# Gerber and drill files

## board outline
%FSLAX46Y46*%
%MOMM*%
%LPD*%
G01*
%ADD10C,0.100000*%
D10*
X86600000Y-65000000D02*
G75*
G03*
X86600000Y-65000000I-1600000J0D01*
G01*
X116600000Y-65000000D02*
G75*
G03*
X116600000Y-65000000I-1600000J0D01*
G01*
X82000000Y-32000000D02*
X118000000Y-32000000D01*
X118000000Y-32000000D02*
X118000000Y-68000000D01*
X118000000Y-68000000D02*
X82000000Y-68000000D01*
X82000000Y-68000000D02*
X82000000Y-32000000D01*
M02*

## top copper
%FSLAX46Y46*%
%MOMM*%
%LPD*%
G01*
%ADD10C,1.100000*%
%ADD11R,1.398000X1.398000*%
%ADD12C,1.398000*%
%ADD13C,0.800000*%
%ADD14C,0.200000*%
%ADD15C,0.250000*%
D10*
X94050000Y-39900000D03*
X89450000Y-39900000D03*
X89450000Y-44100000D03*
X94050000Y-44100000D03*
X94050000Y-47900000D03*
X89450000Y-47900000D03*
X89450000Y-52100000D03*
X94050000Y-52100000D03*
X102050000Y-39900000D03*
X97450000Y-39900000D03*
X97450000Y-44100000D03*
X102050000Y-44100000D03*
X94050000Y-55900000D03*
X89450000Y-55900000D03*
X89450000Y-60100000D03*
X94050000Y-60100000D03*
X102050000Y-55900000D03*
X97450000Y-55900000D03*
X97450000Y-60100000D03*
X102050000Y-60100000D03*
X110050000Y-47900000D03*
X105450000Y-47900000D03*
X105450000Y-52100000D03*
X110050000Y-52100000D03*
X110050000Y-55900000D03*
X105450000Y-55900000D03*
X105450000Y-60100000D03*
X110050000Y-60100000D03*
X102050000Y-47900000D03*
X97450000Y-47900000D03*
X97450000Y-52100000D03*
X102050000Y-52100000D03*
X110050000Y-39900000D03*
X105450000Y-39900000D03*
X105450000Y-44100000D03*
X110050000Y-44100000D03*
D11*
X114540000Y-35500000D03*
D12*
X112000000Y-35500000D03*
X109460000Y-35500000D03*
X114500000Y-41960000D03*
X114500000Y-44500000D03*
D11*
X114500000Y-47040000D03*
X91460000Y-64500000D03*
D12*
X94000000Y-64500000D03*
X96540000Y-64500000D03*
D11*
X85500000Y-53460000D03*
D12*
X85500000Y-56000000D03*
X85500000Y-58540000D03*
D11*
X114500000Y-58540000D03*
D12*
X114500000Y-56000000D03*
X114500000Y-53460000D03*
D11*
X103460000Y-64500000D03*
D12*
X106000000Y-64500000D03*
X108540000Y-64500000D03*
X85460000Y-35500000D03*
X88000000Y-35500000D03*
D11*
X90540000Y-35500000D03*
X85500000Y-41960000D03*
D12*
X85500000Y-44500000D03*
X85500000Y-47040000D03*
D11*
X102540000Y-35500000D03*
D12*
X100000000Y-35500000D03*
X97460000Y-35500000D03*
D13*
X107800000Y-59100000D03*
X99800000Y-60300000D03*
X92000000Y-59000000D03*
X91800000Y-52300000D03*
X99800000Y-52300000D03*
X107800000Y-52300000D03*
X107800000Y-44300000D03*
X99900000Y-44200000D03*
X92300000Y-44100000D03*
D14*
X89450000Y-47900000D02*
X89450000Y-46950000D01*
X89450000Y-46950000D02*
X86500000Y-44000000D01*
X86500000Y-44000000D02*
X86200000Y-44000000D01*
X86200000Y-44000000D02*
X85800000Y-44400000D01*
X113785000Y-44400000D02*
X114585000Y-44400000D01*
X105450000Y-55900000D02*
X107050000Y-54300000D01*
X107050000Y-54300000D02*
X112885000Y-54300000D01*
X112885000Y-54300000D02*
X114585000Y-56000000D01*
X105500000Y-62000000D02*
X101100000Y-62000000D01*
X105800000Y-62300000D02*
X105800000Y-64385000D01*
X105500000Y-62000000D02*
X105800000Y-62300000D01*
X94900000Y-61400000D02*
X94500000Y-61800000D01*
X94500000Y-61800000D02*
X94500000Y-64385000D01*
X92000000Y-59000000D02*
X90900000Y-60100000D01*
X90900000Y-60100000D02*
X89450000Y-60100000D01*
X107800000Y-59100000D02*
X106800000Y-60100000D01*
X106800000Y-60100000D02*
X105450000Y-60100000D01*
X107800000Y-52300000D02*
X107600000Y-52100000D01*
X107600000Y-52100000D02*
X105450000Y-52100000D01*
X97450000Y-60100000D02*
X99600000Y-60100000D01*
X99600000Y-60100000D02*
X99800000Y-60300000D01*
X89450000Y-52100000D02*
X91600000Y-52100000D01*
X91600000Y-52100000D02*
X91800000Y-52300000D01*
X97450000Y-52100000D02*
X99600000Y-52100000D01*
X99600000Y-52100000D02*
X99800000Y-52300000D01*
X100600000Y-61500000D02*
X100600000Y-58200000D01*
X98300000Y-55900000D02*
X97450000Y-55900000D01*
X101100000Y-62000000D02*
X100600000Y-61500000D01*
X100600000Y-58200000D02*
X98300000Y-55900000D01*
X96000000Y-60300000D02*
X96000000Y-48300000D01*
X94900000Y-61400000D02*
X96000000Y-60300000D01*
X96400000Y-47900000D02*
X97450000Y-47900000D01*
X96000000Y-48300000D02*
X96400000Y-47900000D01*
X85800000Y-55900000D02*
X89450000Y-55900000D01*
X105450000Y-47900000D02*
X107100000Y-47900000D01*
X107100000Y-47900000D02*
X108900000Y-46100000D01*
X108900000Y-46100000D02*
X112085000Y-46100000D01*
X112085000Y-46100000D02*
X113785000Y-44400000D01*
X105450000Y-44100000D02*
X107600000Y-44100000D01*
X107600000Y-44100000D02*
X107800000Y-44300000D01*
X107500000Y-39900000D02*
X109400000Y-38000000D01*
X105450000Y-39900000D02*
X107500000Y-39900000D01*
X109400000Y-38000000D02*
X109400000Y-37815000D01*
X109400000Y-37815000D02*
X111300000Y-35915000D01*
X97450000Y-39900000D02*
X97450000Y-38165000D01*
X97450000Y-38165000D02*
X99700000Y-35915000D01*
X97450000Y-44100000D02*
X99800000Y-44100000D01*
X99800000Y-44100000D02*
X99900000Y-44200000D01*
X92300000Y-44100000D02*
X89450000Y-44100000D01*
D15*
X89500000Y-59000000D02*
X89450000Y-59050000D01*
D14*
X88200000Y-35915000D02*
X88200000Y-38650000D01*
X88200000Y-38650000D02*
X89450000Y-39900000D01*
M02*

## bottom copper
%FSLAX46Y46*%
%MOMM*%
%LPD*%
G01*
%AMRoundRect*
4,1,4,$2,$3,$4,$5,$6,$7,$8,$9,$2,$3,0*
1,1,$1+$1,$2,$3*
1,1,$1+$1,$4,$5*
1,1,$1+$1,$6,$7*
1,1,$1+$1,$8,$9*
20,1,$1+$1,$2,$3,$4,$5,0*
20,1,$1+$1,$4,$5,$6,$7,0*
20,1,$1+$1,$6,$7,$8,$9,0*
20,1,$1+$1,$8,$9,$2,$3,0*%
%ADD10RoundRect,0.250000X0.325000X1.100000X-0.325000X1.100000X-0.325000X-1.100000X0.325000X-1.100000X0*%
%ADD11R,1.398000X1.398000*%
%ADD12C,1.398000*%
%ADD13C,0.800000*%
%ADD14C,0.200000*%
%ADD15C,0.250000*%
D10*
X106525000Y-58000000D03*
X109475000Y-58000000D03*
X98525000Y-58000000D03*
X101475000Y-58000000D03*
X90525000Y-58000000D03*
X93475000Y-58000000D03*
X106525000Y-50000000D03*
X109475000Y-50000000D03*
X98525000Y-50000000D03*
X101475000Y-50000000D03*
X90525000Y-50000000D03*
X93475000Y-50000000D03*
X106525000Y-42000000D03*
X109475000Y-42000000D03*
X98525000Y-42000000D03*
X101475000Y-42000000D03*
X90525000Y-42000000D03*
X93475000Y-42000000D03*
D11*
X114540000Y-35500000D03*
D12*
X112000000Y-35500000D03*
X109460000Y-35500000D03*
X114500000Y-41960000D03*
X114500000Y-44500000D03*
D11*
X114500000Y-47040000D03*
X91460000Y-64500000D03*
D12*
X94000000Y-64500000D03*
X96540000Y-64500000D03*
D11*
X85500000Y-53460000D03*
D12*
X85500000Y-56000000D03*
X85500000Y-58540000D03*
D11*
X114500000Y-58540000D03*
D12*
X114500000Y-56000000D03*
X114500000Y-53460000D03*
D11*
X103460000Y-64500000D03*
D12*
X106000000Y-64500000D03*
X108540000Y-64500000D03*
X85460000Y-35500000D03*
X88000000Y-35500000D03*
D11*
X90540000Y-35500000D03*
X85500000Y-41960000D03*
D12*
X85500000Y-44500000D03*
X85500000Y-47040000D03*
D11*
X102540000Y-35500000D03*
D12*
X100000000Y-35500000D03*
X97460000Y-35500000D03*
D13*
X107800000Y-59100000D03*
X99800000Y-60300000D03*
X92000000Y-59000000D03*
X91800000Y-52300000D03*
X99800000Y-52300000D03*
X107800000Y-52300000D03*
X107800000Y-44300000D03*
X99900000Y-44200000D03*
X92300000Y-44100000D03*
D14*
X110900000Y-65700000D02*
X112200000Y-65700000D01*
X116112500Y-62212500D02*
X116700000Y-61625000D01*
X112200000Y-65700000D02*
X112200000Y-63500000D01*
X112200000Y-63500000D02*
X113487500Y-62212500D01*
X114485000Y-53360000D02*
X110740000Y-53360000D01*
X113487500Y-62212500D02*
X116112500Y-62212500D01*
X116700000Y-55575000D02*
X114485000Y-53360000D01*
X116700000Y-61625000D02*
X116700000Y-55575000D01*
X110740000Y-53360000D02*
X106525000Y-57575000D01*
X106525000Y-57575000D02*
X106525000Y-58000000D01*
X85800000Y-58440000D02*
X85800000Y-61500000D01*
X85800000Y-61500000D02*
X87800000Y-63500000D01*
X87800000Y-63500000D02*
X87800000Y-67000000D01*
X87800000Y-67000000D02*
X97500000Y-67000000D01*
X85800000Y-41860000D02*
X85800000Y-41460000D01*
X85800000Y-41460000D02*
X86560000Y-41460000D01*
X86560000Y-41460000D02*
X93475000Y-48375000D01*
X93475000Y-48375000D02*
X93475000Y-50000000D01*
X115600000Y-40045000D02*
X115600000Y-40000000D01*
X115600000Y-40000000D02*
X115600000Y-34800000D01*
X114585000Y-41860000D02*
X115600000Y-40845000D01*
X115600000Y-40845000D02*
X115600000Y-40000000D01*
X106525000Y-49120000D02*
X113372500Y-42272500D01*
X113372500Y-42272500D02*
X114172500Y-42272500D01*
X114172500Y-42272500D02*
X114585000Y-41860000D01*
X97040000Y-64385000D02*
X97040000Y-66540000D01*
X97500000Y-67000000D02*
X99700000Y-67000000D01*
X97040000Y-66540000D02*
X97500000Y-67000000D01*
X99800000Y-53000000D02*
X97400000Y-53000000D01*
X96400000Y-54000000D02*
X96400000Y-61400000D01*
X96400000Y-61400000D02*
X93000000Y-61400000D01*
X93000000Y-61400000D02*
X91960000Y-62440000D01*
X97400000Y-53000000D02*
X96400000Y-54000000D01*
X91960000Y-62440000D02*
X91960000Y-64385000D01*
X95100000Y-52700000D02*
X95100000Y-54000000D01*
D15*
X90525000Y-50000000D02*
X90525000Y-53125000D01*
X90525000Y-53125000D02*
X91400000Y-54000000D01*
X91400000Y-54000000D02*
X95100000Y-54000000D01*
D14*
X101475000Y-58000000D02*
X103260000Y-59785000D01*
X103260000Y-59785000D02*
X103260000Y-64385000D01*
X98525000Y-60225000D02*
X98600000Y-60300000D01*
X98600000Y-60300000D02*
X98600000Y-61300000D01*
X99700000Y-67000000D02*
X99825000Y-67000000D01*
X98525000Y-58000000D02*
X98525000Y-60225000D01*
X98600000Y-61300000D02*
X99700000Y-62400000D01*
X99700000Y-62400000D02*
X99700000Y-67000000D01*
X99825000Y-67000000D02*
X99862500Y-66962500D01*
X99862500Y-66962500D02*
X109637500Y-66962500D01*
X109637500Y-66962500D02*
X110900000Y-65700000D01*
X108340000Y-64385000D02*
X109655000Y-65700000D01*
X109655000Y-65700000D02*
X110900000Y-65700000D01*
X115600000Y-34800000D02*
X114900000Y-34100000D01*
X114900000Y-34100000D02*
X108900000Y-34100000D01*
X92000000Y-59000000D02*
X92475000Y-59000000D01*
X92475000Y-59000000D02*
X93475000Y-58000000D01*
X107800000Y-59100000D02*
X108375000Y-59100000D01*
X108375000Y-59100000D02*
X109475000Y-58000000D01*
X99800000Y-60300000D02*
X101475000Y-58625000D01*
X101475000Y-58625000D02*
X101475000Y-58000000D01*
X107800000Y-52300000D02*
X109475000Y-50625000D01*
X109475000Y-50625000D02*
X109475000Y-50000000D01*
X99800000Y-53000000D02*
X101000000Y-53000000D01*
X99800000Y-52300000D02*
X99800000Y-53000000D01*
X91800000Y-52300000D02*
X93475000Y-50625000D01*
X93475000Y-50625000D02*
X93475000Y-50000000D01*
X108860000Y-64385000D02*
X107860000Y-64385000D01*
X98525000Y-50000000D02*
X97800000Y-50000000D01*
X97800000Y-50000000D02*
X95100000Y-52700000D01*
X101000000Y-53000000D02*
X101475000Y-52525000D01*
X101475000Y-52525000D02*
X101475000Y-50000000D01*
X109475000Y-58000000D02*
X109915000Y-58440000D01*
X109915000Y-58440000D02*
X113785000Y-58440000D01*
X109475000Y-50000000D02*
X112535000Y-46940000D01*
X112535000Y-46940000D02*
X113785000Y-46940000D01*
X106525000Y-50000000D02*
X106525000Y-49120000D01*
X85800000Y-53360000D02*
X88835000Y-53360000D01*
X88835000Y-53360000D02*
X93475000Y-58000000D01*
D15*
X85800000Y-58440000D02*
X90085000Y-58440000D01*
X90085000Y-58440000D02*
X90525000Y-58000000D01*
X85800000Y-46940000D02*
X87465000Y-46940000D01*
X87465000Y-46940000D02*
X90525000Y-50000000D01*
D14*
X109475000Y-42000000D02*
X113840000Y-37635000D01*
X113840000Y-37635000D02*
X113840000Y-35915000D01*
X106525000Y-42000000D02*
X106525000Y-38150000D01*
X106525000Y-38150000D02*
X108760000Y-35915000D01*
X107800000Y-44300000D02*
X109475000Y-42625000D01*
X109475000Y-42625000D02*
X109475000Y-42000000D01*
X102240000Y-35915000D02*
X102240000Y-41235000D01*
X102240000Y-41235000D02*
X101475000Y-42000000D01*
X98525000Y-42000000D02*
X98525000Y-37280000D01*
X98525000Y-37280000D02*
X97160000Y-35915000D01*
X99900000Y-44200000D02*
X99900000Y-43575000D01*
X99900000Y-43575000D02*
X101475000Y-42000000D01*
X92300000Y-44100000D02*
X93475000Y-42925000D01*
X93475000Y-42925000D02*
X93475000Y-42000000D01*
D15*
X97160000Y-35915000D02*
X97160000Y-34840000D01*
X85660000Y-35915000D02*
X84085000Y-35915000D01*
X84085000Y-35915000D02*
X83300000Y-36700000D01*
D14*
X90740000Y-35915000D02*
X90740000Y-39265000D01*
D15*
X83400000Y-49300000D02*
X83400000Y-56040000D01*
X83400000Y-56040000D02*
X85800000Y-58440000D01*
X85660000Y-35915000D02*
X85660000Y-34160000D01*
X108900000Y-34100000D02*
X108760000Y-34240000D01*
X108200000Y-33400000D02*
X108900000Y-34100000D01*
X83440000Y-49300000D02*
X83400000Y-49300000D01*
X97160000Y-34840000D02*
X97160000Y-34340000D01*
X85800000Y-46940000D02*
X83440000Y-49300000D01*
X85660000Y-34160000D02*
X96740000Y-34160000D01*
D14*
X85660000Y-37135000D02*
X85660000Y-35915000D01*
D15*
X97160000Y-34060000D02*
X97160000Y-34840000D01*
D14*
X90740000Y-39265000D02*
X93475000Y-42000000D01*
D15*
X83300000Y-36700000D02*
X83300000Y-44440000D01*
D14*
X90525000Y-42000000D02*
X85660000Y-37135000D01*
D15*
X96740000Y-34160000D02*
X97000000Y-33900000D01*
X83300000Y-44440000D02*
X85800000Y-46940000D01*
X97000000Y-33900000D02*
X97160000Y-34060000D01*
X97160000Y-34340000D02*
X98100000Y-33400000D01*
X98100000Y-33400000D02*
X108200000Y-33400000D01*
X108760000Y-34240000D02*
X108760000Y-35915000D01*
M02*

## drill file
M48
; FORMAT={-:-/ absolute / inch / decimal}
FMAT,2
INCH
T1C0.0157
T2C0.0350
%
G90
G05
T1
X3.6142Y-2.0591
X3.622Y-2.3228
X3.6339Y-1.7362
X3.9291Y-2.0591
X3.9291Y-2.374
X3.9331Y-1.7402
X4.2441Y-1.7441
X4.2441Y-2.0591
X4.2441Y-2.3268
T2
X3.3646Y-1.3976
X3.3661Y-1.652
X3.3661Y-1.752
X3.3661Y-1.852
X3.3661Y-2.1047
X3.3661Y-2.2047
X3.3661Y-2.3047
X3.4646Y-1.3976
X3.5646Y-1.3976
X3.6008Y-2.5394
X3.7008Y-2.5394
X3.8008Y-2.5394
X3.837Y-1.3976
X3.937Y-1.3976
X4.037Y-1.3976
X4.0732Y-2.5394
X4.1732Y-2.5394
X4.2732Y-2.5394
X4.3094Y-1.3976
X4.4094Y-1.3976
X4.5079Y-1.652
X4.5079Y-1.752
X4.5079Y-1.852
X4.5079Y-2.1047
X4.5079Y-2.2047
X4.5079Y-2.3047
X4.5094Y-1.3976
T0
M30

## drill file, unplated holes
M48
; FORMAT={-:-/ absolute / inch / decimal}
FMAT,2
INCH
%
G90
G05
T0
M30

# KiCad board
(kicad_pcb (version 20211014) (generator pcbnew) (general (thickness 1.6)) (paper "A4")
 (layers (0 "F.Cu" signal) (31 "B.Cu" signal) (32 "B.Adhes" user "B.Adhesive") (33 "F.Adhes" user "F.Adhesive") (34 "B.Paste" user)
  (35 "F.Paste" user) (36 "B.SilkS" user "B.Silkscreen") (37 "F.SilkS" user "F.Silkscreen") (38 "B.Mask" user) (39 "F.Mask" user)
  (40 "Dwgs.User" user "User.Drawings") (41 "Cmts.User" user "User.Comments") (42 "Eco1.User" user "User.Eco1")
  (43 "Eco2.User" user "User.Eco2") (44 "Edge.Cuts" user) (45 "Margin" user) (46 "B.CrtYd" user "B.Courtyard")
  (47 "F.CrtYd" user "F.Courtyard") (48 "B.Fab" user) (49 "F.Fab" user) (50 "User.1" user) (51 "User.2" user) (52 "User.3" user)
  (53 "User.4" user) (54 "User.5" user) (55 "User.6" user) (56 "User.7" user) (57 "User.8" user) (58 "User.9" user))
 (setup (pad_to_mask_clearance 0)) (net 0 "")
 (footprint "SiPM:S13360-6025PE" (layer "F.Cu") (at 92 42)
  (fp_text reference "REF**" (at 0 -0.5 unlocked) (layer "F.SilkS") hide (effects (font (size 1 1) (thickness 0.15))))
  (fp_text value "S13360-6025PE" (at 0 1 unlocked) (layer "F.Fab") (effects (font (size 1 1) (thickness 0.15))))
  (pad "1" smd circle (at 2.05 -2.1) (size 1.1 1.1) (layers "F.Cu" "F.Paste" "F.Mask"))
  (pad "2" smd circle (at -2.55 -2.1) (size 1.1 1.1) (layers "F.Cu" "F.Paste" "F.Mask"))
  (pad "3" smd circle (at -2.55 2.1) (size 1.1 1.1) (layers "F.Cu" "F.Paste" "F.Mask"))
  (pad "4" smd circle (at 2.05 2.1) (size 1.1 1.1) (layers "F.Cu" "F.Paste" "F.Mask")))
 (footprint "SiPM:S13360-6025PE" (layer "F.Cu") (at 92 50)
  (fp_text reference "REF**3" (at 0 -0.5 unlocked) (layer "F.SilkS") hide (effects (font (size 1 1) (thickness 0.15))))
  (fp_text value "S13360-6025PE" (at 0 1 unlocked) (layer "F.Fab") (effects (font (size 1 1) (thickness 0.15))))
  (pad "1" smd circle (at 2.05 -2.1) (size 1.1 1.1) (layers "F.Cu" "F.Paste" "F.Mask"))
  (pad "2" smd circle (at -2.55 -2.1) (size 1.1 1.1) (layers "F.Cu" "F.Paste" "F.Mask"))
  (pad "3" smd circle (at -2.55 2.1) (size 1.1 1.1) (layers "F.Cu" "F.Paste" "F.Mask"))
  (pad "4" smd circle (at 2.05 2.1) (size 1.1 1.1) (layers "F.Cu" "F.Paste" "F.Mask")))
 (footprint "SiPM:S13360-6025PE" (layer "F.Cu") (at 100 42)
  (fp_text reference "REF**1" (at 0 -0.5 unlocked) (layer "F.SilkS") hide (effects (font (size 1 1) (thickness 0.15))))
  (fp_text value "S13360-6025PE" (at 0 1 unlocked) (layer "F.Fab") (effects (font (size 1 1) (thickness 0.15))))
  (pad "1" smd circle (at 2.05 -2.1) (size 1.1 1.1) (layers "F.Cu" "F.Paste" "F.Mask"))
  (pad "2" smd circle (at -2.55 -2.1) (size 1.1 1.1) (layers "F.Cu" "F.Paste" "F.Mask"))
  (pad "3" smd circle (at -2.55 2.1) (size 1.1 1.1) (layers "F.Cu" "F.Paste" "F.Mask"))
  (pad "4" smd circle (at 2.05 2.1) (size 1.1 1.1) (layers "F.Cu" "F.Paste" "F.Mask")))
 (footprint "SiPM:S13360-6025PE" (layer "F.Cu") (at 92 58)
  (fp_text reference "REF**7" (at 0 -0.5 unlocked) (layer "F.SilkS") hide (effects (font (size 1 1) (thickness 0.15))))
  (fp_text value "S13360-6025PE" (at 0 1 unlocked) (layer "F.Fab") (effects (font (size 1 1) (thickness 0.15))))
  (pad "1" smd circle (at 2.05 -2.1) (size 1.1 1.1) (layers "F.Cu" "F.Paste" "F.Mask"))
  (pad "2" smd circle (at -2.55 -2.1) (size 1.1 1.1) (layers "F.Cu" "F.Paste" "F.Mask"))
  (pad "3" smd circle (at -2.55 2.1) (size 1.1 1.1) (layers "F.Cu" "F.Paste" "F.Mask"))
  (pad "4" smd circle (at 2.05 2.1) (size 1.1 1.1) (layers "F.Cu" "F.Paste" "F.Mask")))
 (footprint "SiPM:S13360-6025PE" (layer "F.Cu") (at 100 58)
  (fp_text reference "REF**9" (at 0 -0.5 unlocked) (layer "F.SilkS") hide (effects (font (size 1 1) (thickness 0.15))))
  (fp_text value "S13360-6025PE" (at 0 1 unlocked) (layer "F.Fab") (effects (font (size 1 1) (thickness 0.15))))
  (pad "1" smd circle (at 2.05 -2.1) (size 1.1 1.1) (layers "F.Cu" "F.Paste" "F.Mask"))
  (pad "2" smd circle (at -2.55 -2.1) (size 1.1 1.1) (layers "F.Cu" "F.Paste" "F.Mask"))
  (pad "3" smd circle (at -2.55 2.1) (size 1.1 1.1) (layers "F.Cu" "F.Paste" "F.Mask"))
  (pad "4" smd circle (at 2.05 2.1) (size 1.1 1.1) (layers "F.Cu" "F.Paste" "F.Mask")))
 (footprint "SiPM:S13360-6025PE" (layer "F.Cu") (at 108 50)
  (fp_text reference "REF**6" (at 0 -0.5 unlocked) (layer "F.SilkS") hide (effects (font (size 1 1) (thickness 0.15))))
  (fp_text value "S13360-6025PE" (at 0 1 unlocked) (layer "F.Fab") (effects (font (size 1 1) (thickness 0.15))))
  (pad "1" smd circle (at 2.05 -2.1) (size 1.1 1.1) (layers "F.Cu" "F.Paste" "F.Mask"))
  (pad "2" smd circle (at -2.55 -2.1) (size 1.1 1.1) (layers "F.Cu" "F.Paste" "F.Mask"))
  (pad "3" smd circle (at -2.55 2.1) (size 1.1 1.1) (layers "F.Cu" "F.Paste" "F.Mask"))
  (pad "4" smd circle (at 2.05 2.1) (size 1.1 1.1) (layers "F.Cu" "F.Paste" "F.Mask")))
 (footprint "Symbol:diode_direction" (layer "F.Cu") (at 87.3 41.8 90)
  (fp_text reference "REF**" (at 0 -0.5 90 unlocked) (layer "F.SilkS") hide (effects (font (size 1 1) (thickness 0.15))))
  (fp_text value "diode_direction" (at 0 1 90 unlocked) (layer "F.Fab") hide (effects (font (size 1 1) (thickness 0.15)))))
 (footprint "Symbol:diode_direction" (layer "F.Cu") (at 87.3 49.8 90)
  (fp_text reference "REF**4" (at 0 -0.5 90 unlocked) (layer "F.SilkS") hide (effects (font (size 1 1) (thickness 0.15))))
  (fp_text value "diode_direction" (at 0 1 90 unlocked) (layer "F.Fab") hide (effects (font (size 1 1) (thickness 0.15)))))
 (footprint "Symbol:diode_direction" (layer "F.Cu") (at 87.3 57.8 90)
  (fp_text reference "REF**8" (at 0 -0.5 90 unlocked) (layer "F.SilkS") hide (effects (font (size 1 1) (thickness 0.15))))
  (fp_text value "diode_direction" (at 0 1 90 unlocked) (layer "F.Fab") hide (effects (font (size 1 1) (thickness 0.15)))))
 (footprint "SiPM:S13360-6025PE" (layer "F.Cu") (at 108 58)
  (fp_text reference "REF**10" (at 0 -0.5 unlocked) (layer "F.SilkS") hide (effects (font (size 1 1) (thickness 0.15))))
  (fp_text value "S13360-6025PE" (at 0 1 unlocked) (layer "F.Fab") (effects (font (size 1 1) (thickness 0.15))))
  (pad "1" smd circle (at 2.05 -2.1) (size 1.1 1.1) (layers "F.Cu" "F.Paste" "F.Mask"))
  (pad "2" smd circle (at -2.55 -2.1) (size 1.1 1.1) (layers "F.Cu" "F.Paste" "F.Mask"))
  (pad "3" smd circle (at -2.55 2.1) (size 1.1 1.1) (layers "F.Cu" "F.Paste" "F.Mask"))
  (pad "4" smd circle (at 2.05 2.1) (size 1.1 1.1) (layers "F.Cu" "F.Paste" "F.Mask")))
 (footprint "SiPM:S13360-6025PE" (layer "F.Cu") (at 100 50)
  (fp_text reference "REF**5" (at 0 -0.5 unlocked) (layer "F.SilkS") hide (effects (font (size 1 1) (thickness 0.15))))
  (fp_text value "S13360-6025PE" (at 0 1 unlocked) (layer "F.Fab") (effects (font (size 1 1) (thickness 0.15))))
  (pad "1" smd circle (at 2.05 -2.1) (size 1.1 1.1) (layers "F.Cu" "F.Paste" "F.Mask"))
  (pad "2" smd circle (at -2.55 -2.1) (size 1.1 1.1) (layers "F.Cu" "F.Paste" "F.Mask"))
  (pad "3" smd circle (at -2.55 2.1) (size 1.1 1.1) (layers "F.Cu" "F.Paste" "F.Mask"))
  (pad "4" smd circle (at 2.05 2.1) (size 1.1 1.1) (layers "F.Cu" "F.Paste" "F.Mask")))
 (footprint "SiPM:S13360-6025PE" (layer "F.Cu") (at 108 42)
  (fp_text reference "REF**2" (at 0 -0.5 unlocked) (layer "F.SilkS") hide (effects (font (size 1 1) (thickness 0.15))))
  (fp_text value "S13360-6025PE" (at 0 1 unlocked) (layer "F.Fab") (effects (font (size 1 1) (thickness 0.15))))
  (pad "1" smd circle (at 2.05 -2.1) (size 1.1 1.1) (layers "F.Cu" "F.Paste" "F.Mask"))
  (pad "2" smd circle (at -2.55 -2.1) (size 1.1 1.1) (layers "F.Cu" "F.Paste" "F.Mask"))
  (pad "3" smd circle (at -2.55 2.1) (size 1.1 1.1) (layers "F.Cu" "F.Paste" "F.Mask"))
  (pad "4" smd circle (at 2.05 2.1) (size 1.1 1.1) (layers "F.Cu" "F.Paste" "F.Mask")))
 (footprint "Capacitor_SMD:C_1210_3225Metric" (layer "B.Cu") (at 100 58 180)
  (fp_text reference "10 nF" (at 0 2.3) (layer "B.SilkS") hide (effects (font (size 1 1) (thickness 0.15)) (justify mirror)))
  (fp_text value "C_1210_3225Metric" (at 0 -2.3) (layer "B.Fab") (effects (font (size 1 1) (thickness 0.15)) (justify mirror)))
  (pad "1" smd roundrect (at -1.475 0 180) (size 1.15 2.7) (layers "B.Cu" "B.Paste" "B.Mask") (roundrect_rratio 0.2173913043))
  (pad "2" smd roundrect (at 1.475 0 180) (size 1.15 2.7) (layers "B.Cu" "B.Paste" "B.Mask") (roundrect_rratio 0.2173913043)))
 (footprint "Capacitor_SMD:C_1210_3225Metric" (layer "B.Cu") (at 92 42 180)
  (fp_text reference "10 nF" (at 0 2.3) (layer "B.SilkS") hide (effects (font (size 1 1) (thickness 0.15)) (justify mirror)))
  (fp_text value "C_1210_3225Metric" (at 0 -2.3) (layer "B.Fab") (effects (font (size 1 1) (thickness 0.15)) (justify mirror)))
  (pad "1" smd roundrect (at -1.475 0 180) (size 1.15 2.7) (layers "B.Cu" "B.Paste" "B.Mask") (roundrect_rratio 0.2173913043))
  (pad "2" smd roundrect (at 1.475 0 180) (size 1.15 2.7) (layers "B.Cu" "B.Paste" "B.Mask") (roundrect_rratio 0.2173913043)))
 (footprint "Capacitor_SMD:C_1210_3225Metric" (layer "B.Cu") (at 108 58 180)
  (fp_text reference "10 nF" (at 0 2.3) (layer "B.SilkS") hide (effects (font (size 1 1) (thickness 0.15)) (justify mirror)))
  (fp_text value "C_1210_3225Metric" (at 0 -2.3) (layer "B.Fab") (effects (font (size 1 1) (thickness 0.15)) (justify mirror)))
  (pad "1" smd roundrect (at -1.475 0 180) (size 1.15 2.7) (layers "B.Cu" "B.Paste" "B.Mask") (roundrect_rratio 0.2173913043))
  (pad "2" smd roundrect (at 1.475 0 180) (size 1.15 2.7) (layers "B.Cu" "B.Paste" "B.Mask") (roundrect_rratio 0.2173913043)))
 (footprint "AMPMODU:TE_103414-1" (layer "B.Cu") (at 112 35.5 180)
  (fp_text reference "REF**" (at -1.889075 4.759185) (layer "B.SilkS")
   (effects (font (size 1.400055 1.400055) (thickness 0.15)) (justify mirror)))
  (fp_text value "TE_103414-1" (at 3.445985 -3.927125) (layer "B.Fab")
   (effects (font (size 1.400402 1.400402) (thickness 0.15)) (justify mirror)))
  (pad "1" thru_hole rect locked (at -2.54 0 180) (size 1.398 1.398) (drill 0.89) (layers *.Cu *.Mask) (solder_mask_margin 0.102))
  (pad "2" thru_hole circle locked (at 0 0 180) (size 1.398 1.398) (drill 0.89) (layers *.Cu *.Mask) (solder_mask_margin 0.102))
  (pad "3" thru_hole circle locked (at 2.54 0 180) (size 1.398 1.398) (drill 0.89) (layers *.Cu *.Mask) (solder_mask_margin 0.102)))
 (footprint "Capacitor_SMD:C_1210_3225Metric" (layer "B.Cu") (at 108 42 180)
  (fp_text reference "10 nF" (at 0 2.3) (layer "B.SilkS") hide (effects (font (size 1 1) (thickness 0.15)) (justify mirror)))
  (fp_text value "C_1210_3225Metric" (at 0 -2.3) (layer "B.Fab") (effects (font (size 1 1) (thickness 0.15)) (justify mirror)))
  (pad "1" smd roundrect (at -1.475 0 180) (size 1.15 2.7) (layers "B.Cu" "B.Paste" "B.Mask") (roundrect_rratio 0.2173913043))
  (pad "2" smd roundrect (at 1.475 0 180) (size 1.15 2.7) (layers "B.Cu" "B.Paste" "B.Mask") (roundrect_rratio 0.2173913043)))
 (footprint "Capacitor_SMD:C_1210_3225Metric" (layer "B.Cu") (at 92 50 180)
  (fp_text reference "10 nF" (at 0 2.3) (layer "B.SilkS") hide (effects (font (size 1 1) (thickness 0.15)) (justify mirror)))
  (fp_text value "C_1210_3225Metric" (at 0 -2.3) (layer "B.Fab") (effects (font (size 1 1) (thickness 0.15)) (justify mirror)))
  (pad "1" smd roundrect (at -1.475 0 180) (size 1.15 2.7) (layers "B.Cu" "B.Paste" "B.Mask") (roundrect_rratio 0.2173913043))
  (pad "2" smd roundrect (at 1.475 0 180) (size 1.15 2.7) (layers "B.Cu" "B.Paste" "B.Mask") (roundrect_rratio 0.2173913043)))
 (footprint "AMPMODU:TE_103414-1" (layer "B.Cu") (at 114.5 44.5 90)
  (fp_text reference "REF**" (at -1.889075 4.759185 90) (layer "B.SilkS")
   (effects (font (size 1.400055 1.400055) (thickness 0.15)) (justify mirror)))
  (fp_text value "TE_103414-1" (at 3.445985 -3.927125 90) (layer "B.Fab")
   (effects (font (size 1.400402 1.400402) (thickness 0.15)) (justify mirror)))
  (pad "1" thru_hole rect locked (at -2.54 0 90) (size 1.398 1.398) (drill 0.89) (layers *.Cu *.Mask) (solder_mask_margin 0.102))
  (pad "2" thru_hole circle locked (at 0 0 90) (size 1.398 1.398) (drill 0.89) (layers *.Cu *.Mask) (solder_mask_margin 0.102))
  (pad "3" thru_hole circle locked (at 2.54 0 90) (size 1.398 1.398) (drill 0.89) (layers *.Cu *.Mask) (solder_mask_margin 0.102)))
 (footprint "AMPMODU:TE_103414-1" (layer "B.Cu") (at 94 64.5)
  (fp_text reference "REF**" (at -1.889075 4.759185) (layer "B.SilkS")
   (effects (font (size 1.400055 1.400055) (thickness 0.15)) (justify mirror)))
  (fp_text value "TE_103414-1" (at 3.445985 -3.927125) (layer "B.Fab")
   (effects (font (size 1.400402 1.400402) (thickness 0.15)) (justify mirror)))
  (pad "1" thru_hole rect locked (at -2.54 0) (size 1.398 1.398) (drill 0.89) (layers *.Cu *.Mask) (solder_mask_margin 0.102))
  (pad "2" thru_hole circle locked (at 0 0) (size 1.398 1.398) (drill 0.89) (layers *.Cu *.Mask) (solder_mask_margin 0.102))
  (pad "3" thru_hole circle locked (at 2.54 0) (size 1.398 1.398) (drill 0.89) (layers *.Cu *.Mask) (solder_mask_margin 0.102)))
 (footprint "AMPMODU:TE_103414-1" (layer "B.Cu") (at 85.5 56 -90)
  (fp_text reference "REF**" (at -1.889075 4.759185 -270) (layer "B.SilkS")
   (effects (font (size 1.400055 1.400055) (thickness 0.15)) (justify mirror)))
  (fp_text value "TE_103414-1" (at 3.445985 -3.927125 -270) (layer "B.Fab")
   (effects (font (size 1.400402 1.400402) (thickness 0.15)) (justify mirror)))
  (pad "1" thru_hole rect locked (at -2.54 0 270) (size 1.398 1.398) (drill 0.89) (layers *.Cu *.Mask) (solder_mask_margin 0.102))
  (pad "2" thru_hole circle locked (at 0 0 270) (size 1.398 1.398) (drill 0.89) (layers *.Cu *.Mask) (solder_mask_margin 0.102))
  (pad "3" thru_hole circle locked (at 2.54 0 270) (size 1.398 1.398) (drill 0.89) (layers *.Cu *.Mask) (solder_mask_margin 0.102)))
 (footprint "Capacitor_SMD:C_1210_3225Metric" (layer "B.Cu") (at 108 50 180)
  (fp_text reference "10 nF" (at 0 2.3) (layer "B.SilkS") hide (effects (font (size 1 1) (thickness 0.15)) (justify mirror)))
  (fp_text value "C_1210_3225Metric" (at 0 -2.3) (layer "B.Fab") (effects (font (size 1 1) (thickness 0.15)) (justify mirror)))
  (pad "1" smd roundrect (at -1.475 0 180) (size 1.15 2.7) (layers "B.Cu" "B.Paste" "B.Mask") (roundrect_rratio 0.2173913043))
  (pad "2" smd roundrect (at 1.475 0 180) (size 1.15 2.7) (layers "B.Cu" "B.Paste" "B.Mask") (roundrect_rratio 0.2173913043)))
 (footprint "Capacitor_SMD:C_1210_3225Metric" (layer "B.Cu") (at 100 50 180)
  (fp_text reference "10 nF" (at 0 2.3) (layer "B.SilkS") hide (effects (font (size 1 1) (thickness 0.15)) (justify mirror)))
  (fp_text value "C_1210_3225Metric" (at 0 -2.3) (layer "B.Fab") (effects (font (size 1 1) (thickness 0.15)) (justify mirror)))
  (pad "1" smd roundrect (at -1.475 0 180) (size 1.15 2.7) (layers "B.Cu" "B.Paste" "B.Mask") (roundrect_rratio 0.2173913043))
  (pad "2" smd roundrect (at 1.475 0 180) (size 1.15 2.7) (layers "B.Cu" "B.Paste" "B.Mask") (roundrect_rratio 0.2173913043)))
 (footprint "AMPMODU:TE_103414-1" (layer "B.Cu") (at 114.5 56 90)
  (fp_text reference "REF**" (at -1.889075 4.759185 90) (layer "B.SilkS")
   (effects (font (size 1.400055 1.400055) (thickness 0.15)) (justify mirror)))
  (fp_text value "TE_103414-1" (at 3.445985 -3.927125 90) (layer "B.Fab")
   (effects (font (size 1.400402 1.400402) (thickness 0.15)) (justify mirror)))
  (pad "1" thru_hole rect locked (at -2.54 0 90) (size 1.398 1.398) (drill 0.89) (layers *.Cu *.Mask) (solder_mask_margin 0.102))
  (pad "2" thru_hole circle locked (at 0 0 90) (size 1.398 1.398) (drill 0.89) (layers *.Cu *.Mask) (solder_mask_margin 0.102))
  (pad "3" thru_hole circle locked (at 2.54 0 90) (size 1.398 1.398) (drill 0.89) (layers *.Cu *.Mask) (solder_mask_margin 0.102)))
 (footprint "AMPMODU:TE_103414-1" (layer "B.Cu") (at 106 64.5)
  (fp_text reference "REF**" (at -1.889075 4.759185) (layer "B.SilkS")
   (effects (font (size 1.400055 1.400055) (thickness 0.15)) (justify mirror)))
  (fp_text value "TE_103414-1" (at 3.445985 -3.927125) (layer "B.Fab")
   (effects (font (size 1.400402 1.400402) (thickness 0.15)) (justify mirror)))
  (pad "1" thru_hole rect locked (at -2.54 0) (size 1.398 1.398) (drill 0.89) (layers *.Cu *.Mask) (solder_mask_margin 0.102))
  (pad "2" thru_hole circle locked (at 0 0) (size 1.398 1.398) (drill 0.89) (layers *.Cu *.Mask) (solder_mask_margin 0.102))
  (pad "3" thru_hole circle locked (at 2.54 0) (size 1.398 1.398) (drill 0.89) (layers *.Cu *.Mask) (solder_mask_margin 0.102)))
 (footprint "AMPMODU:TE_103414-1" (layer "B.Cu") (at 88 35.5 180)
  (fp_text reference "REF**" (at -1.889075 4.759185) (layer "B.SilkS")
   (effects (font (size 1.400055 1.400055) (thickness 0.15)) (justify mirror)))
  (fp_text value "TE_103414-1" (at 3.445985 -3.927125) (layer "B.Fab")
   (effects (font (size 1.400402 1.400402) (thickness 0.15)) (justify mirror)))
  (pad "1" thru_hole rect locked (at -2.54 0 180) (size 1.398 1.398) (drill 0.89) (layers *.Cu *.Mask) (solder_mask_margin 0.102))
  (pad "2" thru_hole circle locked (at 0 0 180) (size 1.398 1.398) (drill 0.89) (layers *.Cu *.Mask) (solder_mask_margin 0.102))
  (pad "3" thru_hole circle locked (at 2.54 0 180) (size 1.398 1.398) (drill 0.89) (layers *.Cu *.Mask) (solder_mask_margin 0.102)))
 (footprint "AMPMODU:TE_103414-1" (layer "B.Cu") (at 85.5 44.5 -90)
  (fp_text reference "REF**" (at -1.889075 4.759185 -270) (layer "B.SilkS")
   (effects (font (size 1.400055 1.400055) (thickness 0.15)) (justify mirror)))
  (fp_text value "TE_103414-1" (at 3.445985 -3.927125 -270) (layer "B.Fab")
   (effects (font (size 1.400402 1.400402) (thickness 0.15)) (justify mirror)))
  (pad "1" thru_hole rect locked (at -2.54 0 270) (size 1.398 1.398) (drill 0.89) (layers *.Cu *.Mask) (solder_mask_margin 0.102))
  (pad "2" thru_hole circle locked (at 0 0 270) (size 1.398 1.398) (drill 0.89) (layers *.Cu *.Mask) (solder_mask_margin 0.102))
  (pad "3" thru_hole circle locked (at 2.54 0 270) (size 1.398 1.398) (drill 0.89) (layers *.Cu *.Mask) (solder_mask_margin 0.102)))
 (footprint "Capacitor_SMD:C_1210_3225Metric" (layer "B.Cu") (at 92 58 180)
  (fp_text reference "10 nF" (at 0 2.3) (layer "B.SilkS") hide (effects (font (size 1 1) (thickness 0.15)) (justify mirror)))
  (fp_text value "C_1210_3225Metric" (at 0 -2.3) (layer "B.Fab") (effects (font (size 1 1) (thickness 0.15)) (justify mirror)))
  (pad "1" smd roundrect (at -1.475 0 180) (size 1.15 2.7) (layers "B.Cu" "B.Paste" "B.Mask") (roundrect_rratio 0.2173913043))
  (pad "2" smd roundrect (at 1.475 0 180) (size 1.15 2.7) (layers "B.Cu" "B.Paste" "B.Mask") (roundrect_rratio 0.2173913043)))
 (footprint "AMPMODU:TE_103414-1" (layer "B.Cu") (at 100 35.5 180)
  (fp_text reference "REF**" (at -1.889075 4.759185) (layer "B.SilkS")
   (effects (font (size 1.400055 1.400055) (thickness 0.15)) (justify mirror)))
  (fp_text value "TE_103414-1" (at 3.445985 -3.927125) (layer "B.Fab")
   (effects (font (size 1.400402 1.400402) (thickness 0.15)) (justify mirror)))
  (pad "1" thru_hole rect locked (at -2.54 0 180) (size 1.398 1.398) (drill 0.89) (layers *.Cu *.Mask) (solder_mask_margin 0.102))
  (pad "2" thru_hole circle locked (at 0 0 180) (size 1.398 1.398) (drill 0.89) (layers *.Cu *.Mask) (solder_mask_margin 0.102))
  (pad "3" thru_hole circle locked (at 2.54 0 180) (size 1.398 1.398) (drill 0.89) (layers *.Cu *.Mask) (solder_mask_margin 0.102)))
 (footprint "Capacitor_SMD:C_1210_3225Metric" (layer "B.Cu") (at 100 42 180)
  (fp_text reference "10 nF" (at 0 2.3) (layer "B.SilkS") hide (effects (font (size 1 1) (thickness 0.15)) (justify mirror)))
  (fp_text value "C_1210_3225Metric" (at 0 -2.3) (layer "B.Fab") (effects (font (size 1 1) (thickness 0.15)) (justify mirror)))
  (pad "1" smd roundrect (at -1.475 0 180) (size 1.15 2.7) (layers "B.Cu" "B.Paste" "B.Mask") (roundrect_rratio 0.2173913043))
  (pad "2" smd roundrect (at 1.475 0 180) (size 1.15 2.7) (layers "B.Cu" "B.Paste" "B.Mask") (roundrect_rratio 0.2173913043)))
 (gr_rect (start 82 32) (end 118 68) (layer "Edge.Cuts") (width 0.1) (fill none))
 (gr_circle (center 115 65) (end 115 63.4) (layer "Edge.Cuts") (width 0.1) (fill none))
 (gr_circle (center 85 65) (end 85 63.4) (layer "Edge.Cuts") (width 0.1) (fill none))
 (segment (start 92.3 44.1) (end 89.45 44.1) (width 0.2) (layer "F.Cu") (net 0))
 (segment (start 112.885 54.3) (end 114.585 56) (width 0.2) (layer "F.Cu") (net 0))
 (segment (start 100.6 58.2) (end 98.3 55.9) (width 0.2) (layer "F.Cu") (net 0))
 (segment (start 89.5 59) (end 89.45 59.05) (width 0.25) (layer "F.Cu") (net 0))
 (segment (start 97.45 39.9) (end 97.45 38.165) (width 0.2) (layer "F.Cu") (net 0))
 (segment (start 88.2 35.915) (end 88.2 38.65) (width 0.2) (layer "F.Cu") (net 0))
 (segment (start 107.6 52.1) (end 105.45 52.1) (width 0.2) (layer "F.Cu") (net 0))
 (segment (start 107.8 59.1) (end 106.8 60.1) (width 0.2) (layer "F.Cu") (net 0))
 (segment (start 108.9 46.1) (end 112.085 46.1) (width 0.2) (layer "F.Cu") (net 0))
 (segment (start 109.4 37.815) (end 111.3 35.915) (width 0.2) (layer "F.Cu") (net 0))
 (segment (start 96 48.3) (end 96.4 47.9) (width 0.2) (layer "F.Cu") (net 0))
 (segment (start 107.1 47.9) (end 108.9 46.1) (width 0.2) (layer "F.Cu") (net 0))
 (segment (start 107.05 54.3) (end 112.885 54.3) (width 0.2) (layer "F.Cu") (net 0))
 (segment (start 105.8 62.3) (end 105.8 64.385) (width 0.2) (layer "F.Cu") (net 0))
 (segment (start 90.9 60.1) (end 89.45 60.1) (width 0.2) (layer "F.Cu") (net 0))
 (segment (start 98.3 55.9) (end 97.45 55.9) (width 0.2) (layer "F.Cu") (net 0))
 (segment (start 106.8 60.1) (end 105.45 60.1) (width 0.2) (layer "F.Cu") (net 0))
 (segment (start 107.6 44.1) (end 107.8 44.3) (width 0.2) (layer "F.Cu") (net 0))
 (segment (start 97.45 52.1) (end 99.6 52.1) (width 0.2) (layer "F.Cu") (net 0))
 (segment (start 86.2 44) (end 85.8 44.4) (width 0.2) (layer "F.Cu") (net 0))
 (segment (start 94.9 61.4) (end 94.5 61.8) (width 0.2) (layer "F.Cu") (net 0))
 (segment (start 112.085 46.1) (end 113.785 44.4) (width 0.2) (layer "F.Cu") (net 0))
 (segment (start 97.45 44.1) (end 99.8 44.1) (width 0.2) (layer "F.Cu") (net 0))
 (segment (start 94.9 61.4) (end 96 60.3) (width 0.2) (layer "F.Cu") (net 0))
 (segment (start 88.2 38.65) (end 89.45 39.9) (width 0.2) (layer "F.Cu") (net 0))
 (segment (start 105.45 39.9) (end 107.5 39.9) (width 0.2) (layer "F.Cu") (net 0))
 (segment (start 105.5 62) (end 105.8 62.3) (width 0.2) (layer "F.Cu") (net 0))
 (segment (start 99.6 60.1) (end 99.8 60.3) (width 0.2) (layer "F.Cu") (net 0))
 (segment (start 86.5 44) (end 86.2 44) (width 0.2) (layer "F.Cu") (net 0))
 (segment (start 99.6 52.1) (end 99.8 52.3) (width 0.2) (layer "F.Cu") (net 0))
 (segment (start 89.45 47.9) (end 89.45 46.95) (width 0.2) (layer "F.Cu") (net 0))
 (segment (start 97.45 38.165) (end 99.7 35.915) (width 0.2) (layer "F.Cu") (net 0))
 (segment (start 105.5 62) (end 101.1 62) (width 0.2) (layer "F.Cu") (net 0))
 (segment (start 97.45 60.1) (end 99.6 60.1) (width 0.2) (layer "F.Cu") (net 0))
 (segment (start 89.45 46.95) (end 86.5 44) (width 0.2) (layer "F.Cu") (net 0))
 (segment (start 89.45 52.1) (end 91.6 52.1) (width 0.2) (layer "F.Cu") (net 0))
 (segment (start 99.8 44.1) (end 99.9 44.2) (width 0.2) (layer "F.Cu") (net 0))
 (segment (start 101.1 62) (end 100.6 61.5) (width 0.2) (layer "F.Cu") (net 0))
 (segment (start 113.785 44.4) (end 114.585 44.4) (width 0.2) (layer "F.Cu") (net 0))
 (segment (start 92 59) (end 90.9 60.1) (width 0.2) (layer "F.Cu") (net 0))
 (segment (start 105.45 47.9) (end 107.1 47.9) (width 0.2) (layer "F.Cu") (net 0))
 (segment (start 100.6 61.5) (end 100.6 58.2) (width 0.2) (layer "F.Cu") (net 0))
 (segment (start 107.5 39.9) (end 109.4 38) (width 0.2) (layer "F.Cu") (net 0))
 (segment (start 96.4 47.9) (end 97.45 47.9) (width 0.2) (layer "F.Cu") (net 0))
 (segment (start 85.8 55.9) (end 89.45 55.9) (width 0.2) (layer "F.Cu") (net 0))
 (segment (start 105.45 55.9) (end 107.05 54.3) (width 0.2) (layer "F.Cu") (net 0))
 (segment (start 107.8 52.3) (end 107.6 52.1) (width 0.2) (layer "F.Cu") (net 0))
 (segment (start 96 60.3) (end 96 48.3) (width 0.2) (layer "F.Cu") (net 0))
 (segment (start 94.5 61.8) (end 94.5 64.385) (width 0.2) (layer "F.Cu") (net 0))
 (segment (start 105.45 44.1) (end 107.6 44.1) (width 0.2) (layer "F.Cu") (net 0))
 (segment (start 91.6 52.1) (end 91.8 52.3) (width 0.2) (layer "F.Cu") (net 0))
 (segment (start 109.4 38) (end 109.4 37.815) (width 0.2) (layer "F.Cu") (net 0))
 (via (at 92 59) (size 0.8) (drill 0.4) (layers "F.Cu" "B.Cu") (free) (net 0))
 (via (at 92.3 44.1) (size 0.8) (drill 0.4) (layers "F.Cu" "B.Cu") (free) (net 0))
 (via (at 107.8 52.3) (size 0.8) (drill 0.4) (layers "F.Cu" "B.Cu") (free) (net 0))
 (via (at 99.8 52.3) (size 0.8) (drill 0.4) (layers "F.Cu" "B.Cu") (free) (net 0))
 (via (at 107.8 59.1) (size 0.8) (drill 0.4) (layers "F.Cu" "B.Cu") (free) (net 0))
 (via (at 99.9 44.2) (size 0.8) (drill 0.4) (layers "F.Cu" "B.Cu") (free) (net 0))
 (via (at 107.8 44.3) (size 0.8) (drill 0.4) (layers "F.Cu" "B.Cu") (free) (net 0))
 (via (at 91.8 52.3) (size 0.8) (drill 0.4) (layers "F.Cu" "B.Cu") (free) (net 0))
 (via (at 99.8 60.3) (size 0.8) (drill 0.4) (layers "F.Cu" "B.Cu") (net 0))
 (segment (start 95.1 52.7) (end 95.1 54) (width 0.2) (layer "B.Cu") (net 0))
 (segment (start 97.16 35.915) (end 97.16 34.84) (width 0.25) (layer "B.Cu") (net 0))
 (segment (start 113.84 37.635) (end 113.84 35.915) (width 0.2) (layer "B.Cu") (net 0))
 (segment (start 97.8 50) (end 95.1 52.7) (width 0.2) (layer "B.Cu") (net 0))
 (segment (start 99.8 53) (end 101 53) (width 0.2) (layer "B.Cu") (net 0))
 (segment (start 99.7 67) (end 99.825 67) (width 0.2) (layer "B.Cu") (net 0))
 (segment (start 97.4 53) (end 96.4 54) (width 0.2) (layer "B.Cu") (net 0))
 (segment (start 114.485 53.36) (end 110.74 53.36) (width 0.2) (layer "B.Cu") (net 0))
 (segment (start 109.475 50.625) (end 109.475 50) (width 0.2) (layer "B.Cu") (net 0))
 (segment (start 92.475 59) (end 93.475 58) (width 0.2) (layer "B.Cu") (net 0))
 (segment (start 85.66 35.915) (end 84.085 35.915) (width 0.25) (layer "B.Cu") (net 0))
 (segment (start 109.475 42) (end 113.84 37.635) (width 0.2) (layer "B.Cu") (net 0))
 (segment (start 84.085 35.915) (end 83.3 36.7) (width 0.25) (layer "B.Cu") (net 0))
 (segment (start 106.525 38.15) (end 108.76 35.915) (width 0.2) (layer "B.Cu") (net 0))
 (segment (start 90.74 35.915) (end 90.74 39.265) (width 0.2) (layer "B.Cu") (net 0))
 (segment (start 99.825 67) (end 99.8625 66.9625) (width 0.2) (layer "B.Cu") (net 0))
 (segment (start 99.8 60.3) (end 101.475 58.625) (width 0.2) (layer "B.Cu") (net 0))
 (segment (start 102.24 35.915) (end 102.24 41.235) (width 0.2) (layer "B.Cu") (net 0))
 (segment (start 115.6 34.8) (end 114.9 34.1) (width 0.2) (layer "B.Cu") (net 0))
 (segment (start 112.2 63.5) (end 113.4875 62.2125) (width 0.2) (layer "B.Cu") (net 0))
 (segment (start 85.8 58.44) (end 85.8 61.5) (width 0.2) (layer "B.Cu") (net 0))
 (segment (start 87.465 46.94) (end 90.525 50) (width 0.25) (layer "B.Cu") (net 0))
 (segment (start 83.4 49.3) (end 83.4 56.04) (width 0.25) (layer "B.Cu") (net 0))
 (segment (start 83.4 56.04) (end 85.8 58.44) (width 0.25) (layer "B.Cu") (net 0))
 (segment (start 101 53) (end 101.475 52.525) (width 0.2) (layer "B.Cu") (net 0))
 (segment (start 102.24 41.235) (end 101.475 42) (width 0.2) (layer "B.Cu") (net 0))
 (segment (start 109.475 42.625) (end 109.475 42) (width 0.2) (layer "B.Cu") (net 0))
 (segment (start 112.2 65.7) (end 112.2 63.5) (width 0.2) (layer "B.Cu") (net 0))
 (segment (start 109.915 58.44) (end 113.785 58.44) (width 0.2) (layer "B.Cu") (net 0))
 (segment (start 91.4 54) (end 95.1 54) (width 0.25) (layer "B.Cu") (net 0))
 (segment (start 114.585 41.86) (end 115.6 40.845) (width 0.2) (layer "B.Cu") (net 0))
 (segment (start 112.535 46.94) (end 113.785 46.94) (width 0.2) (layer "B.Cu") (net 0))
 (segment (start 99.8 53) (end 97.4 53) (width 0.2) (layer "B.Cu") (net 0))
 (segment (start 85.66 35.915) (end 85.66 34.16) (width 0.25) (layer "B.Cu") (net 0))
 (segment (start 99.8625 66.9625) (end 109.6375 66.9625) (width 0.2) (layer "B.Cu") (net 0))
 (segment (start 97.04 66.54) (end 97.5 67) (width 0.2) (layer "B.Cu") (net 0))
 (segment (start 115.6 40.045) (end 115.6 40) (width 0.2) (layer "B.Cu") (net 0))
 (segment (start 114.9 34.1) (end 108.9 34.1) (width 0.2) (layer "B.Cu") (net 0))
 (segment (start 108.9 34.1) (end 108.76 34.24) (width 0.25) (layer "B.Cu") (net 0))
 (segment (start 98.525 58) (end 98.525 60.225) (width 0.2) (layer "B.Cu") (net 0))
 (segment (start 108.34 64.385) (end 109.655 65.7) (width 0.2) (layer "B.Cu") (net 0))
 (segment (start 101.475 58) (end 103.26 59.785) (width 0.2) (layer "B.Cu") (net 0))
 (segment (start 108.375 59.1) (end 109.475 58) (width 0.2) (layer "B.Cu") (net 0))
 (segment (start 106.525 57.575) (end 106.525 58) (width 0.2) (layer "B.Cu") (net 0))
 (segment (start 108.2 33.4) (end 108.9 34.1) (width 0.25) (layer "B.Cu") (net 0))
 (segment (start 96.4 54) (end 96.4 61.4) (width 0.2) (layer "B.Cu") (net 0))
 (segment (start 101.475 52.525) (end 101.475 50) (width 0.2) (layer "B.Cu") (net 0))
 (segment (start 107.8 59.1) (end 108.375 59.1) (width 0.2) (layer "B.Cu") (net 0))
 (segment (start 109.475 50) (end 112.535 46.94) (width 0.2) (layer "B.Cu") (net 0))
 (segment (start 93.475 48.375) (end 93.475 50) (width 0.2) (layer "B.Cu") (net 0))
 (segment (start 108.86 64.385) (end 107.86 64.385) (width 0.2) (layer "B.Cu") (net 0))
 (segment (start 99.9 43.575) (end 101.475 42) (width 0.2) (layer "B.Cu") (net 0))
 (segment (start 99.7 62.4) (end 99.7 67) (width 0.2) (layer "B.Cu") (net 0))
 (segment (start 83.44 49.3) (end 83.4 49.3) (width 0.25) (layer "B.Cu") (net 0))
 (segment (start 109.655 65.7) (end 110.9 65.7) (width 0.2) (layer "B.Cu") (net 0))
 (segment (start 113.3725 42.2725) (end 114.1725 42.2725) (width 0.2) (layer "B.Cu") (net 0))
 (segment (start 99.9 44.2) (end 99.9 43.575) (width 0.2) (layer "B.Cu") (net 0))
 (segment (start 98.6 60.3) (end 98.6 61.3) (width 0.2) (layer "B.Cu") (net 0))
 (segment (start 93.475 42.925) (end 93.475 42) (width 0.2) (layer "B.Cu") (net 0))
 (segment (start 97.16 34.84) (end 97.16 34.34) (width 0.25) (layer "B.Cu") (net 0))
 (segment (start 88.835 53.36) (end 93.475 58) (width 0.2) (layer "B.Cu") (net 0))
 (segment (start 91.96 62.44) (end 91.96 64.385) (width 0.2) (layer "B.Cu") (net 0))
 (segment (start 85.8 46.94) (end 83.44 49.3) (width 0.25) (layer "B.Cu") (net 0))
 (segment (start 107.8 44.3) (end 109.475 42.625) (width 0.2) (layer "B.Cu") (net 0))
 (segment (start 91.8 52.3) (end 93.475 50.625) (width 0.2) (layer "B.Cu") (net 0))
 (segment (start 85.66 34.16) (end 96.74 34.16) (width 0.25) (layer "B.Cu") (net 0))
 (segment (start 98.6 61.3) (end 99.7 62.4) (width 0.2) (layer "B.Cu") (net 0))
 (segment (start 113.4875 62.2125) (end 116.1125 62.2125) (width 0.2) (layer "B.Cu") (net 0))
 (segment (start 96.4 61.4) (end 93 61.4) (width 0.2) (layer "B.Cu") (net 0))
 (segment (start 87.8 63.5) (end 87.8 67) (width 0.2) (layer "B.Cu") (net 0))
 (segment (start 85.8 46.94) (end 87.465 46.94) (width 0.25) (layer "B.Cu") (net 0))
 (segment (start 110.9 65.7) (end 112.2 65.7) (width 0.2) (layer "B.Cu") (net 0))
 (segment (start 86.56 41.46) (end 93.475 48.375) (width 0.2) (layer "B.Cu") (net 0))
 (segment (start 115.6 40.845) (end 115.6 40) (width 0.2) (layer "B.Cu") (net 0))
 (segment (start 109.6375 66.9625) (end 110.9 65.7) (width 0.2) (layer "B.Cu") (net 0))
 (segment (start 110.74 53.36) (end 106.525 57.575) (width 0.2) (layer "B.Cu") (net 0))
 (segment (start 85.8 41.46) (end 86.56 41.46) (width 0.2) (layer "B.Cu") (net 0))
 (segment (start 85.66 37.135) (end 85.66 35.915) (width 0.2) (layer "B.Cu") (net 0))
 (segment (start 106.525 42) (end 106.525 38.15) (width 0.2) (layer "B.Cu") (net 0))
 (segment (start 85.8 61.5) (end 87.8 63.5) (width 0.2) (layer "B.Cu") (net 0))
 (segment (start 107.8 52.3) (end 109.475 50.625) (width 0.2) (layer "B.Cu") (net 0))
 (segment (start 98.525 37.28) (end 97.16 35.915) (width 0.2) (layer "B.Cu") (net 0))
 (segment (start 116.7 61.625) (end 116.7 55.575) (width 0.2) (layer "B.Cu") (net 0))
 (segment (start 85.8 53.36) (end 88.835 53.36) (width 0.2) (layer "B.Cu") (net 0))
 (segment (start 97.16 34.06) (end 97.16 34.84) (width 0.25) (layer "B.Cu") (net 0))
 (segment (start 90.74 39.265) (end 93.475 42) (width 0.2) (layer "B.Cu") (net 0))
 (segment (start 98.525 42) (end 98.525 37.28) (width 0.2) (layer "B.Cu") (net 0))
 (segment (start 109.475 58) (end 109.915 58.44) (width 0.2) (layer "B.Cu") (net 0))
 (segment (start 92.3 44.1) (end 93.475 42.925) (width 0.2) (layer "B.Cu") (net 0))
 (segment (start 93 61.4) (end 91.96 62.44) (width 0.2) (layer "B.Cu") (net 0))
 (segment (start 85.8 41.86) (end 85.8 41.46) (width 0.2) (layer "B.Cu") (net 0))
 (segment (start 90.525 50) (end 90.525 53.125) (width 0.25) (layer "B.Cu") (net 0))
 (segment (start 83.3 36.7) (end 83.3 44.44) (width 0.25) (layer "B.Cu") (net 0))
 (segment (start 97.04 64.385) (end 97.04 66.54) (width 0.2) (layer "B.Cu") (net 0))
 (segment (start 90.525 42) (end 85.66 37.135) (width 0.2) (layer "B.Cu") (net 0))
 (segment (start 106.525 50) (end 106.525 49.12) (width 0.2) (layer "B.Cu") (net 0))
 (segment (start 116.7 55.575) (end 114.485 53.36) (width 0.2) (layer "B.Cu") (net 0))
 (segment (start 96.74 34.16) (end 97 33.9) (width 0.25) (layer "B.Cu") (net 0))
 (segment (start 83.3 44.44) (end 85.8 46.94) (width 0.25) (layer "B.Cu") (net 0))
 (segment (start 90.085 58.44) (end 90.525 58) (width 0.25) (layer "B.Cu") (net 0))
 (segment (start 116.1125 62.2125) (end 116.7 61.625) (width 0.2) (layer "B.Cu") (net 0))
 (segment (start 97 33.9) (end 97.16 34.06) (width 0.25) (layer "B.Cu") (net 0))
 (segment (start 97.16 34.34) (end 98.1 33.4) (width 0.25) (layer "B.Cu") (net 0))
 (segment (start 98.1 33.4) (end 108.2 33.4) (width 0.25) (layer "B.Cu") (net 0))
 (segment (start 90.525 53.125) (end 91.4 54) (width 0.25) (layer "B.Cu") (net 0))
 (segment (start 103.26 59.785) (end 103.26 64.385) (width 0.2) (layer "B.Cu") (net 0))
 (segment (start 114.1725 42.2725) (end 114.585 41.86) (width 0.2) (layer "B.Cu") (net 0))
 (segment (start 98.525 60.225) (end 98.6 60.3) (width 0.2) (layer "B.Cu") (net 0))
 (segment (start 85.8 58.44) (end 90.085 58.44) (width 0.25) (layer "B.Cu") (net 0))
 (segment (start 115.6 40) (end 115.6 34.8) (width 0.2) (layer "B.Cu") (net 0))
 (segment (start 98.525 50) (end 97.8 50) (width 0.2) (layer "B.Cu") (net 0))
 (segment (start 93.475 50.625) (end 93.475 50) (width 0.2) (layer "B.Cu") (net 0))
 (segment (start 108.76 34.24) (end 108.76 35.915) (width 0.25) (layer "B.Cu") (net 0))
 (segment (start 99.8 52.3) (end 99.8 53) (width 0.2) (layer "B.Cu") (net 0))
 (segment (start 87.8 67) (end 97.5 67) (width 0.2) (layer "B.Cu") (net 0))
 (segment (start 101.475 58.625) (end 101.475 58) (width 0.2) (layer "B.Cu") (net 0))
 (segment (start 106.525 49.12) (end 113.3725 42.2725) (width 0.2) (layer "B.Cu") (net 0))
 (segment (start 92 59) (end 92.475 59) (width 0.2) (layer "B.Cu") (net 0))
 (segment (start 97.5 67) (end 99.7 67) (width 0.2) (layer "B.Cu") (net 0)))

